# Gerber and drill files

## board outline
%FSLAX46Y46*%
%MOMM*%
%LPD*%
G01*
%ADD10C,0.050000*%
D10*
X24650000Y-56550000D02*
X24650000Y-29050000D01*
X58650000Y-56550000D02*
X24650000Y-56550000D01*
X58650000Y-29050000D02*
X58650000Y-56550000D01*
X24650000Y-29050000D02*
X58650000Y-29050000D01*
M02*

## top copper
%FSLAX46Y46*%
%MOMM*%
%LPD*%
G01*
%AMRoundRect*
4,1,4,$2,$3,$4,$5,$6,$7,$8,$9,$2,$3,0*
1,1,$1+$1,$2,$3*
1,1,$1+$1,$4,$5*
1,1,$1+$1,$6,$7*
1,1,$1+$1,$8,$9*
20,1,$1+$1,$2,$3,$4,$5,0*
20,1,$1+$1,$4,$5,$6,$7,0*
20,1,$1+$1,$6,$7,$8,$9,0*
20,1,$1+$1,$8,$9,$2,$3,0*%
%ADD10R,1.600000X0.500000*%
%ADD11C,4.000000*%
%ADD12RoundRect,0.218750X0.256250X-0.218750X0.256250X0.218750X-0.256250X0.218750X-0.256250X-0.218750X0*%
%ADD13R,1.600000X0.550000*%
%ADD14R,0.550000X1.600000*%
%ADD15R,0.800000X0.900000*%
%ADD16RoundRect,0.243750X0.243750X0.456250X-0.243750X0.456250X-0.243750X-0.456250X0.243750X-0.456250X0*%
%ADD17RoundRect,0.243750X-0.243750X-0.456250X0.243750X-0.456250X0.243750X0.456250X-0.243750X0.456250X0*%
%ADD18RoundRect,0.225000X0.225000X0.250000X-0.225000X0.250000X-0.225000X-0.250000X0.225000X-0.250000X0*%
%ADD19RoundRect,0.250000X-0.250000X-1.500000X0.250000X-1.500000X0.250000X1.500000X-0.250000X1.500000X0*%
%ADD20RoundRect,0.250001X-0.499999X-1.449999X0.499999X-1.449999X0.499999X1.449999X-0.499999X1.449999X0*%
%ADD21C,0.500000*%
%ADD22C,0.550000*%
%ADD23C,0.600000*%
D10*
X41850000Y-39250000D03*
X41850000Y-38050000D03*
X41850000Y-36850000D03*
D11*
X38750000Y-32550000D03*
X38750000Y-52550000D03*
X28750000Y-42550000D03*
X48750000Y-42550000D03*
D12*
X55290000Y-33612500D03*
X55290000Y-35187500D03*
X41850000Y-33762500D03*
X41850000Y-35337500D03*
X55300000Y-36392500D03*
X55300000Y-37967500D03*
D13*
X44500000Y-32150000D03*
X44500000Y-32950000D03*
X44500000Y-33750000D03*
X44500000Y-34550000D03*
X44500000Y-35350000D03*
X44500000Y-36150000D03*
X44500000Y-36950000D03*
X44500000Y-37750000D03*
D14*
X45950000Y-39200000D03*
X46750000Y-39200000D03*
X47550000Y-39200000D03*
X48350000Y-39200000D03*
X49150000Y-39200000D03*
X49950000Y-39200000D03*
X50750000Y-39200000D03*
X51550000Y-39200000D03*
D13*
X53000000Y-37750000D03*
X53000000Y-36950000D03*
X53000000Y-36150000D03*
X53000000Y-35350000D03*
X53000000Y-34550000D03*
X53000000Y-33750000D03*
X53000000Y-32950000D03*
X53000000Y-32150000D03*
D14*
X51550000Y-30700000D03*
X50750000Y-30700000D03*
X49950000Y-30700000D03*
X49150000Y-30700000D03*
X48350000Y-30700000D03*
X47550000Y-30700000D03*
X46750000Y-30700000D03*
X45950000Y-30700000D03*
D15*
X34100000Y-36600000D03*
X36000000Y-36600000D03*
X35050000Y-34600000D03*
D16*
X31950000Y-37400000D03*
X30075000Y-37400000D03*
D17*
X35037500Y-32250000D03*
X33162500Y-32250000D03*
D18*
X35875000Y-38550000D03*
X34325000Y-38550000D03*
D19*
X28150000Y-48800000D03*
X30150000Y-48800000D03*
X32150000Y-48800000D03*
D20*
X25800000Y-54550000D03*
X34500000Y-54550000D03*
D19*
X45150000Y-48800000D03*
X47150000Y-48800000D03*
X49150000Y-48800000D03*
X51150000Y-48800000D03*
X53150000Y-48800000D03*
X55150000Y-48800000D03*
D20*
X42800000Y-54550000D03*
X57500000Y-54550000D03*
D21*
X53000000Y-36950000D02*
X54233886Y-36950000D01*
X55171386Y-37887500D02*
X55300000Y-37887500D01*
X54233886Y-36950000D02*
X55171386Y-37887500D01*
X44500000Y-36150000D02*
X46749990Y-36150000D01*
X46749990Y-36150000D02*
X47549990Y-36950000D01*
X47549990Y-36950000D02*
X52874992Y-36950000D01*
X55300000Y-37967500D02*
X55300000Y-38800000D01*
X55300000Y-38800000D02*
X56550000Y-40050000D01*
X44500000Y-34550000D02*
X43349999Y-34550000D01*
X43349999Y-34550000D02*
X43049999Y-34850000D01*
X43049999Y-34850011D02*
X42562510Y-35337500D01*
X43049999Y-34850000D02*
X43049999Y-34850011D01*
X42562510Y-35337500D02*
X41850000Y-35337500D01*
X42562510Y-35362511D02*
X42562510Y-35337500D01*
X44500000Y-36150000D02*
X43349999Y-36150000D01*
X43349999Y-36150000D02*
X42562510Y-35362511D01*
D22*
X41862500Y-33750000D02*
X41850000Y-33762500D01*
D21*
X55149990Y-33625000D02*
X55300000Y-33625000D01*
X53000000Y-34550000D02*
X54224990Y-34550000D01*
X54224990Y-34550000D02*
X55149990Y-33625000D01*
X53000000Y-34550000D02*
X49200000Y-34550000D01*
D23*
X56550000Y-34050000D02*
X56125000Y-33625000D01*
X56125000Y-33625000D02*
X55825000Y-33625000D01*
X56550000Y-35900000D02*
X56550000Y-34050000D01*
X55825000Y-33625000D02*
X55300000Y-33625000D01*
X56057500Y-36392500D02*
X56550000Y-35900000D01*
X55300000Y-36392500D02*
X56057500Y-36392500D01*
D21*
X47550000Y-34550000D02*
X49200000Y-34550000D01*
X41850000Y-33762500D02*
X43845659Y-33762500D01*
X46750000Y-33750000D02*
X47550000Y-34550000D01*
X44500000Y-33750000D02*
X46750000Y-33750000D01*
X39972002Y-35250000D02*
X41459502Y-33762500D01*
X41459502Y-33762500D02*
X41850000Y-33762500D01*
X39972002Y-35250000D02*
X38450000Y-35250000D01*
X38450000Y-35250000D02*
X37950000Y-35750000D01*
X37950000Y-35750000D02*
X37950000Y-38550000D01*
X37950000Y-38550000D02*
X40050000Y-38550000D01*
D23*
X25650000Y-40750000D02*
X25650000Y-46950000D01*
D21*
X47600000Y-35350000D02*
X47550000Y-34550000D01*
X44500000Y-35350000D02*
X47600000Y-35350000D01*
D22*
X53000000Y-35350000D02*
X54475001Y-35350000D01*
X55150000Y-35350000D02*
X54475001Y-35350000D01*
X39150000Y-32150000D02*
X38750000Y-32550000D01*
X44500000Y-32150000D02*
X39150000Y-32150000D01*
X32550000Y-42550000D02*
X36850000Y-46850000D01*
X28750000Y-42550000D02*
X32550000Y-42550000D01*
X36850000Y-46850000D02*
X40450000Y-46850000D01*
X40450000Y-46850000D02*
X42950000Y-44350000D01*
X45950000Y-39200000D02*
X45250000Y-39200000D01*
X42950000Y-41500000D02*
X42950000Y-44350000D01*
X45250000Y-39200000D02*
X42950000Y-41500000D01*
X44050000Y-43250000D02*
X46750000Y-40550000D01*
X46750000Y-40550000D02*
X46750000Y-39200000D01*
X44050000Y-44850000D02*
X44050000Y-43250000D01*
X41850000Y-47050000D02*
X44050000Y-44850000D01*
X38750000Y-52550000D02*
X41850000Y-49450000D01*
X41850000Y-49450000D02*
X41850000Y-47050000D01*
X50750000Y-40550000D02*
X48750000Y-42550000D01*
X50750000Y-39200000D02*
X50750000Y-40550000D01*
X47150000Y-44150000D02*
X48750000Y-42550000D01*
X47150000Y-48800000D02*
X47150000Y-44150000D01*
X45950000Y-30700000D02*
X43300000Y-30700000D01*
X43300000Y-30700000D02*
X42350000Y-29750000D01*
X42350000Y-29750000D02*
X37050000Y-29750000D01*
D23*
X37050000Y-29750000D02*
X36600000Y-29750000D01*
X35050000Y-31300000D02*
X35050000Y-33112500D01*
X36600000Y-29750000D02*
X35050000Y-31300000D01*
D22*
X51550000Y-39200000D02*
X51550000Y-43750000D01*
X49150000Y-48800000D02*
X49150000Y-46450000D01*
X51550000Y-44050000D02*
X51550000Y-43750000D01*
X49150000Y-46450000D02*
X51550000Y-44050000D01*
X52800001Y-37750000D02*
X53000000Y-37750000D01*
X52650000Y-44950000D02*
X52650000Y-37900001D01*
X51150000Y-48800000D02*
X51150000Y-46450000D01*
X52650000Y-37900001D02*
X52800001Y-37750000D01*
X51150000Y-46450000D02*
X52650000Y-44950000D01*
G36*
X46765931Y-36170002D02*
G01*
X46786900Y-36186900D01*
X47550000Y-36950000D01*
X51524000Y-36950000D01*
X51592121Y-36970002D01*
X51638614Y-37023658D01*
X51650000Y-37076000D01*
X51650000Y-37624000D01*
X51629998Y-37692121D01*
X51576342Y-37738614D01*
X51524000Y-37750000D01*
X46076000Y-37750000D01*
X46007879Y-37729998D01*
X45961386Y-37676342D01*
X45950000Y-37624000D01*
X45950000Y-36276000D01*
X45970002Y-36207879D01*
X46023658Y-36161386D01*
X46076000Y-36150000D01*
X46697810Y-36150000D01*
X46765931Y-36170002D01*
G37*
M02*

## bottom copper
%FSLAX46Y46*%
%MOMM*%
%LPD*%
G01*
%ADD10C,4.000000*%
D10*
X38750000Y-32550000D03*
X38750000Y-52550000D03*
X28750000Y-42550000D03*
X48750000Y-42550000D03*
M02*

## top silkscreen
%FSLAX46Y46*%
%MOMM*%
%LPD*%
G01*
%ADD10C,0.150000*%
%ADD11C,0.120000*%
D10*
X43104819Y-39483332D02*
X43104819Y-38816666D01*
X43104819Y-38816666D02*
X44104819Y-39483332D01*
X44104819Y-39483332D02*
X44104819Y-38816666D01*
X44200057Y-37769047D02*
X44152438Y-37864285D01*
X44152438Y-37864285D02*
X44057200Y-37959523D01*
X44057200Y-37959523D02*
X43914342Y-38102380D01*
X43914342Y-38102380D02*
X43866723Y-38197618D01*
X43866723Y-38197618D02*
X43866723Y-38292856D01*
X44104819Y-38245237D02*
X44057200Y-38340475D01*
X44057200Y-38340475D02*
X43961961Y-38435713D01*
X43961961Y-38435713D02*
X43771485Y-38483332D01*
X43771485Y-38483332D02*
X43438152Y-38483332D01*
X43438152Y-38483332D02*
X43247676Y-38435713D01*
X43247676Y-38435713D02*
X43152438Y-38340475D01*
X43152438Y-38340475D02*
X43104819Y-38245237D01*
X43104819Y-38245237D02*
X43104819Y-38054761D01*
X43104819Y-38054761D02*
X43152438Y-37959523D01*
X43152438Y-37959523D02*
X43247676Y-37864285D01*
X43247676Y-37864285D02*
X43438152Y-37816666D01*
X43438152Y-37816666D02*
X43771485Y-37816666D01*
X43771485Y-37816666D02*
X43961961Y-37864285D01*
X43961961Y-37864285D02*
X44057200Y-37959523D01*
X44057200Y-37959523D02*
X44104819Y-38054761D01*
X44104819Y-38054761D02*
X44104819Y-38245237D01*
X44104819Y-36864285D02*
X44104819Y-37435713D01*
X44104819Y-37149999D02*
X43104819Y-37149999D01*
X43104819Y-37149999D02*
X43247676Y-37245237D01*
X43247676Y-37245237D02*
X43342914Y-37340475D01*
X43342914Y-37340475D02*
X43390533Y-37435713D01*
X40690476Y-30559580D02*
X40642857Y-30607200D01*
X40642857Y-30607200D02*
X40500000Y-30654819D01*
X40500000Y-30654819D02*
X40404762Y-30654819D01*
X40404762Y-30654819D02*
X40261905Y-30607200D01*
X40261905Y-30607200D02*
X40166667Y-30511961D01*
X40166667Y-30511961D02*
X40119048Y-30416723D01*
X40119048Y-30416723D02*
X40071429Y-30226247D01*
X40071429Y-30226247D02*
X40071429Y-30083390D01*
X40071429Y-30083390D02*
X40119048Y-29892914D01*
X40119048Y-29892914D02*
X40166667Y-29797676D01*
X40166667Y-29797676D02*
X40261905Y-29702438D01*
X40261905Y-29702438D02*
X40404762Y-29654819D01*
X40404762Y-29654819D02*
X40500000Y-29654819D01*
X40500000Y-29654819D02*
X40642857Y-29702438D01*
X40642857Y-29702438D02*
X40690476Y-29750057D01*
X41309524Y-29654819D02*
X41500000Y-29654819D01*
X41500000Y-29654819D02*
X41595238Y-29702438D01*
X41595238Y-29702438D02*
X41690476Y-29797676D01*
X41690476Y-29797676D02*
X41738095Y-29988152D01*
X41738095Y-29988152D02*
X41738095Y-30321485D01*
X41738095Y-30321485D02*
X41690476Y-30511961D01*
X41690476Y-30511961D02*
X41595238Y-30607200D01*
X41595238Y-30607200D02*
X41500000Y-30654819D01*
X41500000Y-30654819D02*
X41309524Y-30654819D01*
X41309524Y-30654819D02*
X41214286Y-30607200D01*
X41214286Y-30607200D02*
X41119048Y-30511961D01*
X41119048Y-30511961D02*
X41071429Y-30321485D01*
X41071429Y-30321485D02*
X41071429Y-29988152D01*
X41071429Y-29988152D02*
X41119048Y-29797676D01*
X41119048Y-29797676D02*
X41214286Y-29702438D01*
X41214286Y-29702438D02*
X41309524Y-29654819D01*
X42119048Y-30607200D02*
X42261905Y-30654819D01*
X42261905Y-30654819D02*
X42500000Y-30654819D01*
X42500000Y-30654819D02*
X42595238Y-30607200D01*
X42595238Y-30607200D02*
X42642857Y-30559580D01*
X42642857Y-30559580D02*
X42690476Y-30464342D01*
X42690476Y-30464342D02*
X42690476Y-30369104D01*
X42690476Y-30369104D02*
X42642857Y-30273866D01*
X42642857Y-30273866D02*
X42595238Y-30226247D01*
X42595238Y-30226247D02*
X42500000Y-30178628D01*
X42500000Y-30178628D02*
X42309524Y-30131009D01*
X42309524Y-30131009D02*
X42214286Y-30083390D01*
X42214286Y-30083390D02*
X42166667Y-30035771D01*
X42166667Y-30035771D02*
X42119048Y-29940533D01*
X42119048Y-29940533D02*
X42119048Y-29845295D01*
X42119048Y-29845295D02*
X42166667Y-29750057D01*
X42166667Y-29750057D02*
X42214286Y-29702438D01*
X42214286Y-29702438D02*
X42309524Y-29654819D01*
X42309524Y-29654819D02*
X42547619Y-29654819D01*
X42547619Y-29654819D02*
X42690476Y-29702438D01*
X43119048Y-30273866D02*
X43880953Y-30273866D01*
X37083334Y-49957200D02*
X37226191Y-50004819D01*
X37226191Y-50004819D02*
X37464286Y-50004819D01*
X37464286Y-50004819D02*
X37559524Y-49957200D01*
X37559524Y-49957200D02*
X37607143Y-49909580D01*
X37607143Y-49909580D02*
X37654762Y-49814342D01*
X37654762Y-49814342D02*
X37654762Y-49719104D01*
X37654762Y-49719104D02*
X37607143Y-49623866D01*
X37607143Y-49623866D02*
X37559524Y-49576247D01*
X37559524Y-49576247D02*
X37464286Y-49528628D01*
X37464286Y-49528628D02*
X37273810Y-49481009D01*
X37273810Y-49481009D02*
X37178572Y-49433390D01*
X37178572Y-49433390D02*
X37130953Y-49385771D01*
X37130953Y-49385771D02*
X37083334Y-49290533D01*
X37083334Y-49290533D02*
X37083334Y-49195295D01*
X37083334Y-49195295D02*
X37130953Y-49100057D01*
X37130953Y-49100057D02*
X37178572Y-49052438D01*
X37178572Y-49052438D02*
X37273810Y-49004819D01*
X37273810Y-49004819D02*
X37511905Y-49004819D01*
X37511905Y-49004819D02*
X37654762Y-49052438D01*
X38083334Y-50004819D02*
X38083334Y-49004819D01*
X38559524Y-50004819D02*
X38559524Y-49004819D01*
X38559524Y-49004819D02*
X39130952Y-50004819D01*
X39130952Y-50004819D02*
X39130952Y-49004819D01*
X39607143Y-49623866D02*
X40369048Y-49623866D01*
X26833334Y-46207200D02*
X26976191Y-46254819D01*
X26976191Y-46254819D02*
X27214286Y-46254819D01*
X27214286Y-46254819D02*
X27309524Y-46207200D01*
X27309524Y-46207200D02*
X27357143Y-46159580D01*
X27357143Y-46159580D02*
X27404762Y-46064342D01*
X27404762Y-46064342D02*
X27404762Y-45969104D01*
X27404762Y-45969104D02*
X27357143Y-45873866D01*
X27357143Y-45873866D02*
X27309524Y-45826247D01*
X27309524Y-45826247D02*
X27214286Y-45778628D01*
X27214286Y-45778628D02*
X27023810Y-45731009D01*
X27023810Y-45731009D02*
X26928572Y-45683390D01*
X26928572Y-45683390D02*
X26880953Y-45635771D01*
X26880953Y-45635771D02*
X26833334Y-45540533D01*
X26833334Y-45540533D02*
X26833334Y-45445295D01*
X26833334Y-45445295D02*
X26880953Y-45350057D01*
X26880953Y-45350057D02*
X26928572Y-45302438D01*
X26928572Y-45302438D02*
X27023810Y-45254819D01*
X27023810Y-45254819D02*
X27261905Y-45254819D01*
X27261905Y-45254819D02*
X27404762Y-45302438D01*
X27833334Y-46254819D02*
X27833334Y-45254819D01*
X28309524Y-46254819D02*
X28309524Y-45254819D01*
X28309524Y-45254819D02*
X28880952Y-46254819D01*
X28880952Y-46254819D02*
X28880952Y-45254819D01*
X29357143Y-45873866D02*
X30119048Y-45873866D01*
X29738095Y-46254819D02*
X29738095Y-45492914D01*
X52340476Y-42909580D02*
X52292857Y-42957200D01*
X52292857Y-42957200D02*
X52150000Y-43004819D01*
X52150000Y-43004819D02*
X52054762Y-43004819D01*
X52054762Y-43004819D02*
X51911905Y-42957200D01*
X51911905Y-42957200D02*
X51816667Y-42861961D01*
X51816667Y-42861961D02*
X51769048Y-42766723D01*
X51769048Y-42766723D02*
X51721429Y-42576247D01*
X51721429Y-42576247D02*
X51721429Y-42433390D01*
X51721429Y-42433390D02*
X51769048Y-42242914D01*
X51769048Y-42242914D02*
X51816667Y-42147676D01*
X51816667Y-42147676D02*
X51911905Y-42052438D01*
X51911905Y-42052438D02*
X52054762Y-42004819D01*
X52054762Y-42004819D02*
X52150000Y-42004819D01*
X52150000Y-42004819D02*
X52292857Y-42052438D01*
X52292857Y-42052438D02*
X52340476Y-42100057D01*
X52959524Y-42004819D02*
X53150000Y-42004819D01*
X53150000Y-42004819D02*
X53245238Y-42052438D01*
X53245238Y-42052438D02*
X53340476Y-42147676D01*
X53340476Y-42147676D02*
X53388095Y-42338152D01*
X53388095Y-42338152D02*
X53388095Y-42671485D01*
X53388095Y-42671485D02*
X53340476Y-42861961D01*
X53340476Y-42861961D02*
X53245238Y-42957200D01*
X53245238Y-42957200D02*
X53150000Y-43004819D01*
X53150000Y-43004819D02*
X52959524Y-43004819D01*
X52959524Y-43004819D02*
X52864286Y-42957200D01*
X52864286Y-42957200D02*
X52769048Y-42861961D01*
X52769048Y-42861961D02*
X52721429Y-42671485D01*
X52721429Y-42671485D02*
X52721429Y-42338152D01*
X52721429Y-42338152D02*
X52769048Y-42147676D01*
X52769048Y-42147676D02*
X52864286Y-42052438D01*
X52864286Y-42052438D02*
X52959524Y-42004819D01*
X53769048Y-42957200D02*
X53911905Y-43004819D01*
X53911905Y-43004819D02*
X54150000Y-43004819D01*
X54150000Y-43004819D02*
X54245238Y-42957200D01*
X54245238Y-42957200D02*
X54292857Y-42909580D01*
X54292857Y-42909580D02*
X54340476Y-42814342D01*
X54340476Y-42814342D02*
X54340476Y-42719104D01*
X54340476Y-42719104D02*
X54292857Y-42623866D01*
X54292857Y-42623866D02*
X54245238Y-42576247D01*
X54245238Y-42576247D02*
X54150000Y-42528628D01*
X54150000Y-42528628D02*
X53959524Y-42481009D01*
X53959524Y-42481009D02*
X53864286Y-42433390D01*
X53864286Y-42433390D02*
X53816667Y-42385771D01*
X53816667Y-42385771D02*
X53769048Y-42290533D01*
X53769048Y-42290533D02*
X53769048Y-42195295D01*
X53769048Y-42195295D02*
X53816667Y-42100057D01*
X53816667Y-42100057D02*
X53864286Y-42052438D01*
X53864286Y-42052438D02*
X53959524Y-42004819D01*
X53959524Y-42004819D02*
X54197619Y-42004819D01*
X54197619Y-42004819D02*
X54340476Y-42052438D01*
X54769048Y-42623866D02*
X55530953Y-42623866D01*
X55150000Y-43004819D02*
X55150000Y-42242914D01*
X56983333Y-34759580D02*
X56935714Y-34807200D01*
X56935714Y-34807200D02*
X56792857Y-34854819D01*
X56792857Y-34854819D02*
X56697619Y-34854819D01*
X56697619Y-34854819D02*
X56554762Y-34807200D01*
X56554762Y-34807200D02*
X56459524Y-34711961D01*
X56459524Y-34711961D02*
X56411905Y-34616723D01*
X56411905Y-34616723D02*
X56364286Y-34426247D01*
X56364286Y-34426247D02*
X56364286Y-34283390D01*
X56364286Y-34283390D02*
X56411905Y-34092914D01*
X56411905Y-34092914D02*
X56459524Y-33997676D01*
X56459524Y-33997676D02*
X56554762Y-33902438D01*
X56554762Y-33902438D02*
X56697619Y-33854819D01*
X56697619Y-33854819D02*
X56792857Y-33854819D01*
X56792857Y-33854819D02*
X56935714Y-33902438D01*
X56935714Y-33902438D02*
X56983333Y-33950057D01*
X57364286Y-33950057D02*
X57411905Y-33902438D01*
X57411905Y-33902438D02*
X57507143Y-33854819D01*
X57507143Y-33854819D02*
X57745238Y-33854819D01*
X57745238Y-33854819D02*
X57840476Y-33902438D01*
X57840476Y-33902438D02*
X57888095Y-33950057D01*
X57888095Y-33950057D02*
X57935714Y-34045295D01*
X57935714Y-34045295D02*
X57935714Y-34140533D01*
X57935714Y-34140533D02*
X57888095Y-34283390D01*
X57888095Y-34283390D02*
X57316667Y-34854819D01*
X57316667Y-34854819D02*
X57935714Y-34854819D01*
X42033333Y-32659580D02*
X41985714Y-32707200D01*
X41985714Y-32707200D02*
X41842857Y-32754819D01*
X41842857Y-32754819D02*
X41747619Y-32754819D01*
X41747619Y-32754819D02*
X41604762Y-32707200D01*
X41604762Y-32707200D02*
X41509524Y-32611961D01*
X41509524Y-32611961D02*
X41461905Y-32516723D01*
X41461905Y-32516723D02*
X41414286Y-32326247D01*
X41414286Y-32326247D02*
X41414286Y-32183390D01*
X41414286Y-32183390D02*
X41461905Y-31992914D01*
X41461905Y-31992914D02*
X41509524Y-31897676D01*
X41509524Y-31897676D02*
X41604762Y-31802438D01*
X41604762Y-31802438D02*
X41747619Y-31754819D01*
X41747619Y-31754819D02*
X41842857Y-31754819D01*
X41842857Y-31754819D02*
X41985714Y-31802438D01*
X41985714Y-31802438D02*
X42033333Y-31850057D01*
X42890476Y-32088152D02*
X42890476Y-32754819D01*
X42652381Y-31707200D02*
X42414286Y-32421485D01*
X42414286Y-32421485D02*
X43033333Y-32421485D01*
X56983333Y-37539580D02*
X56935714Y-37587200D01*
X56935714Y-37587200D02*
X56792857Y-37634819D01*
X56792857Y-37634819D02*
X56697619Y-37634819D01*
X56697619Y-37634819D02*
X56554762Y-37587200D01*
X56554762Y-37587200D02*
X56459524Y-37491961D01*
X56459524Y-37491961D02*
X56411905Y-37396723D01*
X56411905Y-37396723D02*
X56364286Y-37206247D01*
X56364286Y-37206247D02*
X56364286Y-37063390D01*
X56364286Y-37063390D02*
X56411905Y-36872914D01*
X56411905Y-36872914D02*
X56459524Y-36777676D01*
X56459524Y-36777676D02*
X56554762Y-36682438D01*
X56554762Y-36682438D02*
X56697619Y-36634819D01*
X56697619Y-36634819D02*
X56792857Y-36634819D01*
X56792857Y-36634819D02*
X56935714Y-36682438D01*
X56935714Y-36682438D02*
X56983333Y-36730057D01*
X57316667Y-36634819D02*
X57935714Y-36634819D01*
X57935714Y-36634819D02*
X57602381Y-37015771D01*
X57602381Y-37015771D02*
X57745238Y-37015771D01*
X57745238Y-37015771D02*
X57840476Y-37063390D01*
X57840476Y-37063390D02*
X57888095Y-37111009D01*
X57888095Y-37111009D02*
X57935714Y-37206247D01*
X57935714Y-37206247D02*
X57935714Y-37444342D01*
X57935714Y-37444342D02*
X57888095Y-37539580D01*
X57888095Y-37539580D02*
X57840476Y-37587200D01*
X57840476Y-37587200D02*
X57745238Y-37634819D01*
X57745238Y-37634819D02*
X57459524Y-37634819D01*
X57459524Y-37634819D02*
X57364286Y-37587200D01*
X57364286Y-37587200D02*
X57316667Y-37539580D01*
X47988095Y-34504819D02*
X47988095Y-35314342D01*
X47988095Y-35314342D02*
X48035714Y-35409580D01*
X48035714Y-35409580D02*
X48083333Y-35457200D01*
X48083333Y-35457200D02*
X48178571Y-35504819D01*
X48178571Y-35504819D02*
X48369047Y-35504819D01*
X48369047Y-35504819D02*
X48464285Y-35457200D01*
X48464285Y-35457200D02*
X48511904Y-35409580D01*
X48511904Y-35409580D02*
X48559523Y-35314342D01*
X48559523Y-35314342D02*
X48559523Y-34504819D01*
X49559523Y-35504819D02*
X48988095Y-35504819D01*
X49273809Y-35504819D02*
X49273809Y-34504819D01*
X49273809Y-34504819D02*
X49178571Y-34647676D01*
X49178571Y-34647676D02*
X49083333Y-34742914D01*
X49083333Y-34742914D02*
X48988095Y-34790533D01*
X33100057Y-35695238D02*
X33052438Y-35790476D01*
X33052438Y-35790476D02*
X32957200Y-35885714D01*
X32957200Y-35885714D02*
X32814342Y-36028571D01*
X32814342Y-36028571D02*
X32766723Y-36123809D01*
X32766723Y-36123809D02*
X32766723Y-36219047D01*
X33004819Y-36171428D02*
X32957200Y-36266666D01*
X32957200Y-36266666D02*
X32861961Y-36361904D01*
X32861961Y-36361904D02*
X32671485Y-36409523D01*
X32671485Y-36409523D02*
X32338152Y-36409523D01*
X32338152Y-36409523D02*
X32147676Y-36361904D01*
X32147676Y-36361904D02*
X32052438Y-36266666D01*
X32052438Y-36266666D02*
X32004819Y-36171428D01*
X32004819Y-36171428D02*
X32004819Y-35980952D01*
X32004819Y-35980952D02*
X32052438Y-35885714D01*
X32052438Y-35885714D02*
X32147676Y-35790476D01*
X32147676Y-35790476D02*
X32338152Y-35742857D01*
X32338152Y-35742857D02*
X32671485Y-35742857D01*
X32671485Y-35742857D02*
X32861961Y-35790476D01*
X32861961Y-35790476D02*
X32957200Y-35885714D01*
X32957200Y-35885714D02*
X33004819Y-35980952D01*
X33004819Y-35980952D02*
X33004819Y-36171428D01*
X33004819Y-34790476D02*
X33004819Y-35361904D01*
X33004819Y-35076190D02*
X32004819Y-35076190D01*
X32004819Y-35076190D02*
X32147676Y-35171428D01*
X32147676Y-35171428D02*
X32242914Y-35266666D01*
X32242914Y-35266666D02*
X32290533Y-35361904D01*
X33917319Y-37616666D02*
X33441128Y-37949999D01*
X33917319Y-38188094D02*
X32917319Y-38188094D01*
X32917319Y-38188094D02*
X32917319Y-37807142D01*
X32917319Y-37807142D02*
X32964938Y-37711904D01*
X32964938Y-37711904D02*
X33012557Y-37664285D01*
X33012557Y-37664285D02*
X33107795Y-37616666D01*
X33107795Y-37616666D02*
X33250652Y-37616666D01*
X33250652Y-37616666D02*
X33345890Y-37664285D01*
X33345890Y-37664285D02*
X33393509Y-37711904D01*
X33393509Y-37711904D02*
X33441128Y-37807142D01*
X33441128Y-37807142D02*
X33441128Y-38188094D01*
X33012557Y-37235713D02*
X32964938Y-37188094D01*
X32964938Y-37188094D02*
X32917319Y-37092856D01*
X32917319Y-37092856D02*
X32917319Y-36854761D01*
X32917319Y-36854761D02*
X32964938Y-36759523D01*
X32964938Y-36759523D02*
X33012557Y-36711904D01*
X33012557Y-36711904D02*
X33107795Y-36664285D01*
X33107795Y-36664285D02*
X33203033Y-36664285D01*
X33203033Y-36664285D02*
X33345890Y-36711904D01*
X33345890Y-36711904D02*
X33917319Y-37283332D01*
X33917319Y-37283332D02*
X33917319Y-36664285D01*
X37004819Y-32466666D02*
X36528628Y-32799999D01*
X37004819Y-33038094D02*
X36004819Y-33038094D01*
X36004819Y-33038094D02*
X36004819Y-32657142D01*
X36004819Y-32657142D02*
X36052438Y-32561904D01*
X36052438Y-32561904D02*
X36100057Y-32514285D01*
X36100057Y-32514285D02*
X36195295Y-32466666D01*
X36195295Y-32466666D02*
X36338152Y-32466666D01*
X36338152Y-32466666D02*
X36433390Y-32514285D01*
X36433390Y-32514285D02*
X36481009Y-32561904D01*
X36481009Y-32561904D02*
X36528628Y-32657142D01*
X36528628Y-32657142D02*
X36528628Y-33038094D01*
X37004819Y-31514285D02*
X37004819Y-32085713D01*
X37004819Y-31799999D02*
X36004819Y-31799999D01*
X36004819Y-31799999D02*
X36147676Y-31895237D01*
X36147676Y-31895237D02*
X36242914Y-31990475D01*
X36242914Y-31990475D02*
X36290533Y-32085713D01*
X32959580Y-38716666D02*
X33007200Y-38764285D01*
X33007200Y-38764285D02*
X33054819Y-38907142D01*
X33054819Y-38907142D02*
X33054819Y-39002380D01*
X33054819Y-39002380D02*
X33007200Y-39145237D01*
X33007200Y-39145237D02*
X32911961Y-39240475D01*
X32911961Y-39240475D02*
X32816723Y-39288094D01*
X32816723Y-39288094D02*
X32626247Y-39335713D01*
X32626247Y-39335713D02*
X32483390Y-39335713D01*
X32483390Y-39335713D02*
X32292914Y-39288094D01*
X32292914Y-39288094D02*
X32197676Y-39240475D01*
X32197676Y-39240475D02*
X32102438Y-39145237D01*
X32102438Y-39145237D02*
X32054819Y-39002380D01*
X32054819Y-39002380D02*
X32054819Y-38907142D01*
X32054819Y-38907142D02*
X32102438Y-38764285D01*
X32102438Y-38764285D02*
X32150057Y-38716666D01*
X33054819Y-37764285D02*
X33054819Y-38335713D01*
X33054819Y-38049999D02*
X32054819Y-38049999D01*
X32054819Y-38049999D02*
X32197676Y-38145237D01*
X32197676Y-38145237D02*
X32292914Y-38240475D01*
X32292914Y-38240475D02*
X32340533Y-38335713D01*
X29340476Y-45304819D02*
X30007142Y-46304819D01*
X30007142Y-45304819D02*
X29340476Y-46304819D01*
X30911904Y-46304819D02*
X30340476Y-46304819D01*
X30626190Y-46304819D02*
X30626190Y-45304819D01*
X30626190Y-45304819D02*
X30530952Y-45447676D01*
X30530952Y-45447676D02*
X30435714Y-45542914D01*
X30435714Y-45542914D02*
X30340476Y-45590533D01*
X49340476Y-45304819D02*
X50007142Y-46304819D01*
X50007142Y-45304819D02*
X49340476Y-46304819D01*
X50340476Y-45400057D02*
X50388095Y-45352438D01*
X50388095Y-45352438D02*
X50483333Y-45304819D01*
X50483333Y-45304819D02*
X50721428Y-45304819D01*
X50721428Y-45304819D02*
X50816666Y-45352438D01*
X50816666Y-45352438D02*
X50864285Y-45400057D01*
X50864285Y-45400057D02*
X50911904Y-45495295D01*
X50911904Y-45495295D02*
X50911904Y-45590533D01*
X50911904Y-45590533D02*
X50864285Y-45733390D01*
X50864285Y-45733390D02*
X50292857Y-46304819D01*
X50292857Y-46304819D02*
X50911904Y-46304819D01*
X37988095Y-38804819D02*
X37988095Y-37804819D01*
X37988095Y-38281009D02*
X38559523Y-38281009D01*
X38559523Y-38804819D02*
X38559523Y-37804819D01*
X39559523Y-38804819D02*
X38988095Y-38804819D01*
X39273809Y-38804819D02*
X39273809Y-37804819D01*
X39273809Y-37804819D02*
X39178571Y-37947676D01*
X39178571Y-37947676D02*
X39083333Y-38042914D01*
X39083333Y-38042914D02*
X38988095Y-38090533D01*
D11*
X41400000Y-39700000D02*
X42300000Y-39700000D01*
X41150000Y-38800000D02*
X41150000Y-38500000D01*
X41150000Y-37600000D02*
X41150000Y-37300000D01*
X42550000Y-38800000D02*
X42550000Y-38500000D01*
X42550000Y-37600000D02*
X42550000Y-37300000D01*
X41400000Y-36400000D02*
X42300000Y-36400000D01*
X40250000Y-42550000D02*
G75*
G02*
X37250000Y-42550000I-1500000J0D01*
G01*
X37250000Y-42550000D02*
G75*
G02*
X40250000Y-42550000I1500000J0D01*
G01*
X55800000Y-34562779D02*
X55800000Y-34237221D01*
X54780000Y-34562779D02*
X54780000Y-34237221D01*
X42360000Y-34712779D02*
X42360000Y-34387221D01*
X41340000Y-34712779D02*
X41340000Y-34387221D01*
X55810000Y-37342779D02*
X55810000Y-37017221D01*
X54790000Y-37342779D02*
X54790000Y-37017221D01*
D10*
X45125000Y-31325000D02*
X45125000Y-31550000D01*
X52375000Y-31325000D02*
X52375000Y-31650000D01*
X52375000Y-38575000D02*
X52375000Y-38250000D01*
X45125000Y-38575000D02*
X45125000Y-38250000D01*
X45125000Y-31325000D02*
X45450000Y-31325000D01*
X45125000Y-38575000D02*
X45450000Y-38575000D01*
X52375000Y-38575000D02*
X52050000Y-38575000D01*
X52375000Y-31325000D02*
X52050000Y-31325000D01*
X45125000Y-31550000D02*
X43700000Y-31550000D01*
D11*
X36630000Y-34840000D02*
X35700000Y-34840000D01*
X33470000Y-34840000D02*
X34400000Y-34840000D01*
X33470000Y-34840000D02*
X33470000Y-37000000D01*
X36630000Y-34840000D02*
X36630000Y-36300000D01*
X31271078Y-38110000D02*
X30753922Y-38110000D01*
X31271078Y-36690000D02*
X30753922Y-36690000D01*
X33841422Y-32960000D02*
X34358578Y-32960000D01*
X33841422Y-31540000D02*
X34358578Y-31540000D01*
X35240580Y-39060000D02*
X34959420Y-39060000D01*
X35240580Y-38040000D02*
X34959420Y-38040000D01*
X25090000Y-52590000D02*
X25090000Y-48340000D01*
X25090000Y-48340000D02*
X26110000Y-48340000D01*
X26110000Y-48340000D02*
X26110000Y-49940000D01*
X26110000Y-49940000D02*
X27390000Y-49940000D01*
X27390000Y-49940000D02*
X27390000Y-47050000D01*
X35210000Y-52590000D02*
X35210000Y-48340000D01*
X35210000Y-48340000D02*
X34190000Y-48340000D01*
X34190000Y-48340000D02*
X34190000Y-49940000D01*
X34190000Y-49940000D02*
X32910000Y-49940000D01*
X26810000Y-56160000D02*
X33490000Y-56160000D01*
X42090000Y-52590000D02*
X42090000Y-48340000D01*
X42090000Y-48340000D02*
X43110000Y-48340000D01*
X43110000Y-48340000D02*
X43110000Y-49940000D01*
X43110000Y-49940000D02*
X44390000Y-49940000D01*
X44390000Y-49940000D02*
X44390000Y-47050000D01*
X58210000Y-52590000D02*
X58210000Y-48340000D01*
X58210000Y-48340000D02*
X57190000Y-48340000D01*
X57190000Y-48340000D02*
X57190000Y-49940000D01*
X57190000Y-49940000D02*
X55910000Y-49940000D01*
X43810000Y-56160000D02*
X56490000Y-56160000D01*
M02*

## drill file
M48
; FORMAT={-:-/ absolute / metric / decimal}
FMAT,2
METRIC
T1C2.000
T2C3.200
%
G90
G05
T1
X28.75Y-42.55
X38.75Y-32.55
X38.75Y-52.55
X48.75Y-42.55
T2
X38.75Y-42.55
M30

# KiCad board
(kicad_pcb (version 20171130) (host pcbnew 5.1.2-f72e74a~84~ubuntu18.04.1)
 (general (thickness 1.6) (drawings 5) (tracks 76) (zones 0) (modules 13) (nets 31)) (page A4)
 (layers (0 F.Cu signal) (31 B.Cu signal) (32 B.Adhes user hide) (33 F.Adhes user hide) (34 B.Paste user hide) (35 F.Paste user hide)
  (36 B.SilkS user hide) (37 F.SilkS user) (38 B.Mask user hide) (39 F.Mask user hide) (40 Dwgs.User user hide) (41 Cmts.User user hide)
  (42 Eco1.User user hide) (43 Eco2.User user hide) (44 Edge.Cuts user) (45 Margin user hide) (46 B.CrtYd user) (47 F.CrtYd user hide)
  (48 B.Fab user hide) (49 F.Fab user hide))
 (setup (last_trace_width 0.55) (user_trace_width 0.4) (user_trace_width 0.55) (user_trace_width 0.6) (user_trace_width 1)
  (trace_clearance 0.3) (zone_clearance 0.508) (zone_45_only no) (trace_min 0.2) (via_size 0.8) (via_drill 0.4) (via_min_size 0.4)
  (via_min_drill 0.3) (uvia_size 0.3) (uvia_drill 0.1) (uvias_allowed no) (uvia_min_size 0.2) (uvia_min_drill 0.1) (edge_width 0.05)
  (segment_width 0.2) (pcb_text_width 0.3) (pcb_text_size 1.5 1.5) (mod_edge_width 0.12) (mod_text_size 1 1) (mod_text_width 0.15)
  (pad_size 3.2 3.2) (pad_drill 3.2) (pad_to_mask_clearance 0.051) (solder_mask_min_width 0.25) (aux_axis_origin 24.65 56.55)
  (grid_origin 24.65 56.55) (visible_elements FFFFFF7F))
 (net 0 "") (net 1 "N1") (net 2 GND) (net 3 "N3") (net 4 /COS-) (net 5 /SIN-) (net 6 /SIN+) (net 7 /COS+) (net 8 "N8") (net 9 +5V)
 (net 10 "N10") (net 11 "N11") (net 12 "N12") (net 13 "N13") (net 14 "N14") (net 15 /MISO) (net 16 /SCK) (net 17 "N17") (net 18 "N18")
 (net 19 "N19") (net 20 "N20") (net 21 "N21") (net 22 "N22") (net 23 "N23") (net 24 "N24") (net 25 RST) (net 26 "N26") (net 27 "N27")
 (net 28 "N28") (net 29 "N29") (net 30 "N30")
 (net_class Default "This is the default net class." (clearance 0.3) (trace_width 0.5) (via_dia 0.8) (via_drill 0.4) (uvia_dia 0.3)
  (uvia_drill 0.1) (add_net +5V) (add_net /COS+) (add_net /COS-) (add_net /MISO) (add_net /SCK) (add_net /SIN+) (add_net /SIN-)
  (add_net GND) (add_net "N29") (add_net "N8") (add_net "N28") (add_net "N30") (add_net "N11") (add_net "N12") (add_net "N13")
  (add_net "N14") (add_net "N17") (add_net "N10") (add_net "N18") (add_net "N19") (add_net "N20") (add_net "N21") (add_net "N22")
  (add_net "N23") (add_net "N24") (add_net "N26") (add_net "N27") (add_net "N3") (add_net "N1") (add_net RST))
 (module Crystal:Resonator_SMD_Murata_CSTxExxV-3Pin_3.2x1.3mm (layer F.Cu) (at 41.85 38.05 270)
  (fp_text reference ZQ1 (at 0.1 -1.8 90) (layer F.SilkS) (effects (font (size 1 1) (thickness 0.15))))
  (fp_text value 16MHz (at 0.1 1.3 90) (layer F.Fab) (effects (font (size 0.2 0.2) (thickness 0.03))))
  (fp_line (start 1.65 0.45) (end 1.65 -0.45) (layer F.SilkS) (width 0.12))
  (fp_line (start 0.75 0.7) (end 0.45 0.7) (layer F.SilkS) (width 0.12))
  (fp_line (start -0.45 0.7) (end -0.75 0.7) (layer F.SilkS) (width 0.12))
  (fp_line (start 0.75 -0.7) (end 0.45 -0.7) (layer F.SilkS) (width 0.12))
  (fp_line (start -0.45 -0.7) (end -0.75 -0.7) (layer F.SilkS) (width 0.12))
  (fp_line (start -1.65 0.45) (end -1.65 -0.45) (layer F.SilkS) (width 0.12))
  (pad 3 smd rect (at 1.2 0 270) (size 0.5 1.6) (layers F.Cu F.Paste F.Mask) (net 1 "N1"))
  (pad 2 smd rect (at 0 0 270) (size 0.5 1.6) (layers F.Cu F.Paste F.Mask) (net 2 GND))
  (pad 1 smd rect (at -1.2 0 270) (size 0.5 1.6) (layers F.Cu F.Paste F.Mask) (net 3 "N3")))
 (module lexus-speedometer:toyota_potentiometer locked (layer F.Cu) (at 38.75 42.55)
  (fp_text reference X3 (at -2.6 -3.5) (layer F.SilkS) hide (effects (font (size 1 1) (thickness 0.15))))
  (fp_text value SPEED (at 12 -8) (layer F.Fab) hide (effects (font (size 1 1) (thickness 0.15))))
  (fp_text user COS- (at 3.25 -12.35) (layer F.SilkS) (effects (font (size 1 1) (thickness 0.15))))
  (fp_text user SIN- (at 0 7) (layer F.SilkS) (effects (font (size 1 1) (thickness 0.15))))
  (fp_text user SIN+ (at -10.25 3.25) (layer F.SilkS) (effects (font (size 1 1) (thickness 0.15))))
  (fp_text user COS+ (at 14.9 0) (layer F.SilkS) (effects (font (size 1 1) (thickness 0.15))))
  (fp_circle (center 0 0) (end 1.5 0) (layer F.SilkS) (width 0.12))
  (pad 4 thru_hole circle (at 0 -10) (size 4 4) (drill 2) (layers F.Cu F.Mask) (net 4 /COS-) (clearance 0.6))
  (pad 2 thru_hole circle (at 0 10) (size 4 4) (drill 2) (layers F.Cu F.Mask) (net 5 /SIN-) (clearance 0.6))
  (pad 1 thru_hole circle (at -10 0) (size 4 4) (drill 2) (layers F.Cu F.Mask) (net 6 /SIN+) (clearance 0.6))
  (pad 3 thru_hole circle (at 10 0) (size 4 4) (drill 2) (layers F.Cu F.Mask) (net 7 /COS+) (clearance 0.6)))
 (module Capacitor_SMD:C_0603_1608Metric (layer F.Cu) (at 55.29 34.4 90)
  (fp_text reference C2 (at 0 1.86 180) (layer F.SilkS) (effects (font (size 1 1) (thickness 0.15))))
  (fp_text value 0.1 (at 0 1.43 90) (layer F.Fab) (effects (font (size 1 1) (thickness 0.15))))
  (fp_line (start -0.162779 0.51) (end 0.162779 0.51) (layer F.SilkS) (width 0.12))
  (fp_line (start -0.162779 -0.51) (end 0.162779 -0.51) (layer F.SilkS) (width 0.12))
  (pad 2 smd roundrect (at 0.7875 0 90) (size 0.875 0.95) (layers F.Cu F.Paste F.Mask) (roundrect_rratio 0.25) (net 2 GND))
  (pad 1 smd roundrect (at -0.7875 0 90) (size 0.875 0.95) (layers F.Cu F.Paste F.Mask) (roundrect_rratio 0.25) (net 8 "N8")))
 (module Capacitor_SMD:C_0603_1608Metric (layer F.Cu) (at 41.85 34.55 90)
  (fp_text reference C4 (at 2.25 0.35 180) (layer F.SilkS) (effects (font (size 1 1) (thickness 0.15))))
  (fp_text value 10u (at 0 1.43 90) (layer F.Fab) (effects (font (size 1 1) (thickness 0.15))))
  (fp_line (start -0.162779 0.51) (end 0.162779 0.51) (layer F.SilkS) (width 0.12))
  (fp_line (start -0.162779 -0.51) (end 0.162779 -0.51) (layer F.SilkS) (width 0.12))
  (pad 2 smd roundrect (at 0.7875 0 90) (size 0.875 0.95) (layers F.Cu F.Paste F.Mask) (roundrect_rratio 0.25) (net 2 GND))
  (pad 1 smd roundrect (at -0.7875 0 90) (size 0.875 0.95) (layers F.Cu F.Paste F.Mask) (roundrect_rratio 0.25) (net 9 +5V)))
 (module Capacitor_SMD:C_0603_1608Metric (layer F.Cu) (at 55.3 37.18 90)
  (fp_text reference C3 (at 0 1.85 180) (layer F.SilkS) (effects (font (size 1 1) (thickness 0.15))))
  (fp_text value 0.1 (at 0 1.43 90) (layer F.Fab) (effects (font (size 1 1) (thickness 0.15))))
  (fp_line (start -0.162779 0.51) (end 0.162779 0.51) (layer F.SilkS) (width 0.12))
  (fp_line (start -0.162779 -0.51) (end 0.162779 -0.51) (layer F.SilkS) (width 0.12))
  (pad 2 smd roundrect (at 0.7875 0 90) (size 0.875 0.95) (layers F.Cu F.Paste F.Mask) (roundrect_rratio 0.25) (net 2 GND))
  (pad 1 smd roundrect (at -0.7875 0 90) (size 0.875 0.95) (layers F.Cu F.Paste F.Mask) (roundrect_rratio 0.25) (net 9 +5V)))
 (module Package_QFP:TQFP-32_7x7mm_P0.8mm (layer F.Cu) (at 48.75 34.95)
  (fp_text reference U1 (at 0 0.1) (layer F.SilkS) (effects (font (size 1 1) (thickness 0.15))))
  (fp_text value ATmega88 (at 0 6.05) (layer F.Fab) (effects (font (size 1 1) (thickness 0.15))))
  (fp_line (start -3.625 -3.625) (end -3.625 -3.4) (layer F.SilkS) (width 0.15))
  (fp_line (start 3.625 -3.625) (end 3.625 -3.3) (layer F.SilkS) (width 0.15))
  (fp_line (start 3.625 3.625) (end 3.625 3.3) (layer F.SilkS) (width 0.15))
  (fp_line (start -3.625 3.625) (end -3.625 3.3) (layer F.SilkS) (width 0.15))
  (fp_line (start -3.625 -3.625) (end -3.3 -3.625) (layer F.SilkS) (width 0.15))
  (fp_line (start -3.625 3.625) (end -3.3 3.625) (layer F.SilkS) (width 0.15))
  (fp_line (start 3.625 3.625) (end 3.3 3.625) (layer F.SilkS) (width 0.15))
  (fp_line (start 3.625 -3.625) (end 3.3 -3.625) (layer F.SilkS) (width 0.15))
  (fp_line (start -3.625 -3.4) (end -5.05 -3.4) (layer F.SilkS) (width 0.15))
  (pad 1 smd rect (at -4.25 -2.8) (size 1.6 0.55) (layers F.Cu F.Paste F.Mask) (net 4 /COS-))
  (pad 2 smd rect (at -4.25 -2) (size 1.6 0.55) (layers F.Cu F.Paste F.Mask) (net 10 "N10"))
  (pad 3 smd rect (at -4.25 -1.2) (size 1.6 0.55) (layers F.Cu F.Paste F.Mask) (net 2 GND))
  (pad 4 smd rect (at -4.25 -0.4) (size 1.6 0.55) (layers F.Cu F.Paste F.Mask) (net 9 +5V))
  (pad 5 smd rect (at -4.25 0.4) (size 1.6 0.55) (layers F.Cu F.Paste F.Mask) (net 2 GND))
  (pad 6 smd rect (at -4.25 1.2) (size 1.6 0.55) (layers F.Cu F.Paste F.Mask) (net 9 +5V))
  (pad 7 smd rect (at -4.25 2) (size 1.6 0.55) (layers F.Cu F.Paste F.Mask) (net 3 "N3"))
  (pad 8 smd rect (at -4.25 2.8) (size 1.6 0.55) (layers F.Cu F.Paste F.Mask) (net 1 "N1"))
  (pad 9 smd rect (at -2.8 4.25 90) (size 1.6 0.55) (layers F.Cu F.Paste F.Mask) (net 6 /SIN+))
  (pad 10 smd rect (at -2 4.25 90) (size 1.6 0.55) (layers F.Cu F.Paste F.Mask) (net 5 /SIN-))
  (pad 11 smd rect (at -1.2 4.25 90) (size 1.6 0.55) (layers F.Cu F.Paste F.Mask) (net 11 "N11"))
  (pad 12 smd rect (at -0.4 4.25 90) (size 1.6 0.55) (layers F.Cu F.Paste F.Mask) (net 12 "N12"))
  (pad 13 smd rect (at 0.4 4.25 90) (size 1.6 0.55) (layers F.Cu F.Paste F.Mask) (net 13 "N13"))
  (pad 14 smd rect (at 1.2 4.25 90) (size 1.6 0.55) (layers F.Cu F.Paste F.Mask) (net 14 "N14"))
  (pad 15 smd rect (at 2 4.25 90) (size 1.6 0.55) (layers F.Cu F.Paste F.Mask) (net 7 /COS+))
  (pad 16 smd rect (at 2.8 4.25 90) (size 1.6 0.55) (layers F.Cu F.Paste F.Mask) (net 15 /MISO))
  (pad 17 smd rect (at 4.25 2.8) (size 1.6 0.55) (layers F.Cu F.Paste F.Mask) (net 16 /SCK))
  (pad 18 smd rect (at 4.25 2) (size 1.6 0.55) (layers F.Cu F.Paste F.Mask) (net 9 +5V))
  (pad 19 smd rect (at 4.25 1.2) (size 1.6 0.55) (layers F.Cu F.Paste F.Mask) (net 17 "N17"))
  (pad 20 smd rect (at 4.25 0.4) (size 1.6 0.55) (layers F.Cu F.Paste F.Mask) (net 8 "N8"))
  (pad 21 smd rect (at 4.25 -0.4) (size 1.6 0.55) (layers F.Cu F.Paste F.Mask) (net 2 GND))
  (pad 22 smd rect (at 4.25 -1.2) (size 1.6 0.55) (layers F.Cu F.Paste F.Mask) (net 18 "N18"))
  (pad 23 smd rect (at 4.25 -2) (size 1.6 0.55) (layers F.Cu F.Paste F.Mask) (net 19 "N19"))
  (pad 24 smd rect (at 4.25 -2.8) (size 1.6 0.55) (layers F.Cu F.Paste F.Mask) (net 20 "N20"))
  (pad 25 smd rect (at 2.8 -4.25 90) (size 1.6 0.55) (layers F.Cu F.Paste F.Mask) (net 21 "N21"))
  (pad 26 smd rect (at 2 -4.25 90) (size 1.6 0.55) (layers F.Cu F.Paste F.Mask) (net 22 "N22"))
  (pad 27 smd rect (at 1.2 -4.25 90) (size 1.6 0.55) (layers F.Cu F.Paste F.Mask) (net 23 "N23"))
  (pad 28 smd rect (at 0.4 -4.25 90) (size 1.6 0.55) (layers F.Cu F.Paste F.Mask) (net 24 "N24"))
  (pad 29 smd rect (at -0.4 -4.25 90) (size 1.6 0.55) (layers F.Cu F.Paste F.Mask) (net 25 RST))
  (pad 30 smd rect (at -1.2 -4.25 90) (size 1.6 0.55) (layers F.Cu F.Paste F.Mask) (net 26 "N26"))
  (pad 31 smd rect (at -2 -4.25 90) (size 1.6 0.55) (layers F.Cu F.Paste F.Mask) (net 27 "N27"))
  (pad 32 smd rect (at -2.8 -4.25 90) (size 1.6 0.55) (layers F.Cu F.Paste F.Mask) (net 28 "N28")))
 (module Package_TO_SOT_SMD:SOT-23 (layer F.Cu) (at 35.05 35.6 90)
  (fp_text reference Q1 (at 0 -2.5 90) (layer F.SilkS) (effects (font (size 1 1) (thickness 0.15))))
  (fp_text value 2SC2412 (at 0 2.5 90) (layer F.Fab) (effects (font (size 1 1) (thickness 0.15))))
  (fp_line (start 0.76 1.58) (end 0.76 0.65) (layer F.SilkS) (width 0.12))
  (fp_line (start 0.76 -1.58) (end 0.76 -0.65) (layer F.SilkS) (width 0.12))
  (fp_line (start 0.76 -1.58) (end -1.4 -1.58) (layer F.SilkS) (width 0.12))
  (fp_line (start 0.76 1.58) (end -0.7 1.58) (layer F.SilkS) (width 0.12))
  (pad 1 smd rect (at -1 -0.95 90) (size 0.9 0.8) (layers F.Cu F.Paste F.Mask) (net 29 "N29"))
  (pad 2 smd rect (at -1 0.95 90) (size 0.9 0.8) (layers F.Cu F.Paste F.Mask) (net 2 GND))
  (pad 3 smd rect (at 1 0 90) (size 0.9 0.8) (layers F.Cu F.Paste F.Mask) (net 28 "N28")))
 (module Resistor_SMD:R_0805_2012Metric (layer F.Cu) (at 31.0125 37.4 180)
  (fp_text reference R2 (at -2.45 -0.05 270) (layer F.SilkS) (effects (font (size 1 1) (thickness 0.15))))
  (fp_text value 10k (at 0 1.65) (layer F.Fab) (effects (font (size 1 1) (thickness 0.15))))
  (fp_line (start -0.258578 -0.71) (end 0.258578 -0.71) (layer F.SilkS) (width 0.12))
  (fp_line (start -0.258578 0.71) (end 0.258578 0.71) (layer F.SilkS) (width 0.12))
  (pad 1 smd roundrect (at -0.9375 0 180) (size 0.975 1.4) (layers F.Cu F.Paste F.Mask) (roundrect_rratio 0.25) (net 29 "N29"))
  (pad 2 smd roundrect (at 0.9375 0 180) (size 0.975 1.4) (layers F.Cu F.Paste F.Mask) (roundrect_rratio 0.25) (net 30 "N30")))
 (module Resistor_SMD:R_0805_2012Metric (layer F.Cu) (at 34.1 32.25)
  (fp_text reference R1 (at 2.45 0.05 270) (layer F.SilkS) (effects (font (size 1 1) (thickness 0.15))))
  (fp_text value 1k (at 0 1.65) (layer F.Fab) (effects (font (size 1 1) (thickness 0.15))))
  (fp_line (start -0.258578 0.71) (end 0.258578 0.71) (layer F.SilkS) (width 0.12))
  (fp_line (start -0.258578 -0.71) (end 0.258578 -0.71) (layer F.SilkS) (width 0.12))
  (pad 2 smd roundrect (at 0.9375 0) (size 0.975 1.4) (layers F.Cu F.Paste F.Mask) (roundrect_rratio 0.25) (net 28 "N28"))
  (pad 1 smd roundrect (at -0.9375 0) (size 0.975 1.4) (layers F.Cu F.Paste F.Mask) (roundrect_rratio 0.25) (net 9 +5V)))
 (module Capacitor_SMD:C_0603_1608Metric (layer F.Cu) (at 35.1 38.55 180)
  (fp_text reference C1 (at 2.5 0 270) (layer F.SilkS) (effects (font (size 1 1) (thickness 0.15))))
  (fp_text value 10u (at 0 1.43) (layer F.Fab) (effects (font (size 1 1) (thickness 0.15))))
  (fp_line (start -0.14058 -0.51) (end 0.14058 -0.51) (layer F.SilkS) (width 0.12))
  (fp_line (start -0.14058 0.51) (end 0.14058 0.51) (layer F.SilkS) (width 0.12))
  (pad 1 smd roundrect (at -0.775 0 180) (size 0.9 0.95) (layers F.Cu F.Paste F.Mask) (roundrect_rratio 0.25) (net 2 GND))
  (pad 2 smd roundrect (at 0.775 0 180) (size 0.9 0.95) (layers F.Cu F.Paste F.Mask) (roundrect_rratio 0.25) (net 29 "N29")))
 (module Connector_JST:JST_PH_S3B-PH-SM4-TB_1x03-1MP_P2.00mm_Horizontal (layer F.Cu) (at 30.15 51.65)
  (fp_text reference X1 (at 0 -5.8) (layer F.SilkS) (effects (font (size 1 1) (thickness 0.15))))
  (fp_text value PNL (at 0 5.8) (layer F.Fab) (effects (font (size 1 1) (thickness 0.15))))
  (fp_line (start -5.06 0.94) (end -5.06 -3.31) (layer F.SilkS) (width 0.12))
  (fp_line (start -5.06 -3.31) (end -4.04 -3.31) (layer F.SilkS) (width 0.12))
  (fp_line (start -4.04 -3.31) (end -4.04 -1.71) (layer F.SilkS) (width 0.12))
  (fp_line (start -4.04 -1.71) (end -2.76 -1.71) (layer F.SilkS) (width 0.12))
  (fp_line (start -2.76 -1.71) (end -2.76 -4.6) (layer F.SilkS) (width 0.12))
  (fp_line (start 5.06 0.94) (end 5.06 -3.31) (layer F.SilkS) (width 0.12))
  (fp_line (start 5.06 -3.31) (end 4.04 -3.31) (layer F.SilkS) (width 0.12))
  (fp_line (start 4.04 -3.31) (end 4.04 -1.71) (layer F.SilkS) (width 0.12))
  (fp_line (start 4.04 -1.71) (end 2.76 -1.71) (layer F.SilkS) (width 0.12))
  (fp_line (start -3.34 4.51) (end 3.34 4.51) (layer F.SilkS) (width 0.12))
  (pad 1 smd roundrect (at -2 -2.85) (size 1 3.5) (layers F.Cu F.Paste F.Mask) (roundrect_rratio 0.25) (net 2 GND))
  (pad 2 smd roundrect (at 0 -2.85) (size 1 3.5) (layers F.Cu F.Paste F.Mask) (roundrect_rratio 0.25) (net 30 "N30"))
  (pad 3 smd roundrect (at 2 -2.85) (size 1 3.5) (layers F.Cu F.Paste F.Mask) (roundrect_rratio 0.25) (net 9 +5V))
  (pad MP smd roundrect (at -4.35 2.9) (size 1.5 3.4) (layers F.Cu F.Paste F.Mask) (roundrect_rratio 0.166667))
  (pad MP smd roundrect (at 4.35 2.9) (size 1.5 3.4) (layers F.Cu F.Paste F.Mask) (roundrect_rratio 0.166667)))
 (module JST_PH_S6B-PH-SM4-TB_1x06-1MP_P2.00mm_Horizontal (layer F.Cu) (at 50.15 51.65)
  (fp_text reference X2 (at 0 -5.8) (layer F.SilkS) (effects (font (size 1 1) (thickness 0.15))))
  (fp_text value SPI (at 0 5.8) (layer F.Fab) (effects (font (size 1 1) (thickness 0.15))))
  (fp_line (start -8.06 0.94) (end -8.06 -3.31) (layer F.SilkS) (width 0.12))
  (fp_line (start -8.06 -3.31) (end -7.04 -3.31) (layer F.SilkS) (width 0.12))
  (fp_line (start -7.04 -3.31) (end -7.04 -1.71) (layer F.SilkS) (width 0.12))
  (fp_line (start -7.04 -1.71) (end -5.76 -1.71) (layer F.SilkS) (width 0.12))
  (fp_line (start -5.76 -1.71) (end -5.76 -4.6) (layer F.SilkS) (width 0.12))
  (fp_line (start 8.06 0.94) (end 8.06 -3.31) (layer F.SilkS) (width 0.12))
  (fp_line (start 8.06 -3.31) (end 7.04 -3.31) (layer F.SilkS) (width 0.12))
  (fp_line (start 7.04 -3.31) (end 7.04 -1.71) (layer F.SilkS) (width 0.12))
  (fp_line (start 7.04 -1.71) (end 5.76 -1.71) (layer F.SilkS) (width 0.12))
  (fp_line (start -6.34 4.51) (end 6.34 4.51) (layer F.SilkS) (width 0.12))
  (pad 1 smd roundrect (at -5 -2.85) (size 1 3.5) (layers F.Cu F.Paste F.Mask) (roundrect_rratio 0.25) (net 2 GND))
  (pad 2 smd roundrect (at -3 -2.85) (size 1 3.5) (layers F.Cu F.Paste F.Mask) (roundrect_rratio 0.25) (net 7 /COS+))
  (pad 3 smd roundrect (at -1 -2.85) (size 1 3.5) (layers F.Cu F.Paste F.Mask) (roundrect_rratio 0.25) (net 15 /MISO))
  (pad 4 smd roundrect (at 1 -2.85) (size 1 3.5) (layers F.Cu F.Paste F.Mask) (roundrect_rratio 0.25) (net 16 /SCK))
  (pad 5 smd roundrect (at 3 -2.85) (size 1 3.5) (layers F.Cu F.Paste F.Mask) (roundrect_rratio 0.25) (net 25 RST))
  (pad 6 smd roundrect (at 5 -2.85) (size 1 3.5) (layers F.Cu F.Paste F.Mask) (roundrect_rratio 0.25) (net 9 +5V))
  (pad MP smd roundrect (at -7.35 2.9) (size 1.5 3.4) (layers F.Cu F.Paste F.Mask) (roundrect_rratio 0.166667))
  (pad MP smd roundrect (at 7.35 2.9) (size 1.5 3.4) (layers F.Cu F.Paste F.Mask) (roundrect_rratio 0.166667)))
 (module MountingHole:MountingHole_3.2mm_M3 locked (layer F.Cu) (at 38.75 42.55) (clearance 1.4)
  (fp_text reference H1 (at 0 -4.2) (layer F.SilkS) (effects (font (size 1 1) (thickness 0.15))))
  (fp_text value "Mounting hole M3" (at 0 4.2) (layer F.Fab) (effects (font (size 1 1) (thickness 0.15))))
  (pad 1 np_thru_hole circle (at 0 0) (size 3.2 3.2) (drill 3.2) (layers *.Cu *.Mask)))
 (gr_line (start 24.65 56.55) (end 24.65 29.05) (layer Edge.Cuts) (width 0.05))
 (gr_line (start 58.65 56.55) (end 24.65 56.55) (layer Edge.Cuts) (width 0.05))
 (gr_line (start 58.65 29.05) (end 58.65 56.55) (layer Edge.Cuts) (width 0.05))
 (gr_line (start 24.65 29.05) (end 58.65 29.05) (layer Edge.Cuts) (width 0.05))
 (segment (start 53 36.95) (end 54.233886 36.95) (width 0.5) (layer F.Cu) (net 9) (status 10))
 (segment (start 55.171386 37.8875) (end 55.3 37.8875) (width 0.5) (layer F.Cu) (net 9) (status 30))
 (segment (start 54.233886 36.95) (end 55.171386 37.8875) (width 0.5) (layer F.Cu) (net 9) (status 20))
 (segment (start 44.5 36.15) (end 46.74999 36.15) (width 0.5) (layer F.Cu) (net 9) (status 10))
 (segment (start 46.74999 36.15) (end 47.54999 36.95) (width 0.5) (layer F.Cu) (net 9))
 (segment (start 47.54999 36.95) (end 52.874992 36.95) (width 0.5) (layer F.Cu) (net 9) (status 20))
 (segment (start 55.3 37.9675) (end 55.3 38.8) (width 0.5) (layer F.Cu) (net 9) (status 10))
 (segment (start 55.3 38.8) (end 56.55 40.05) (width 0.5) (layer F.Cu) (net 9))
 (segment (start 44.5 34.55) (end 43.349999 34.55) (width 0.5) (layer F.Cu) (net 9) (status 10))
 (segment (start 43.349999 34.55) (end 43.049999 34.85) (width 0.5) (layer F.Cu) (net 9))
 (segment (start 43.049999 34.850011) (end 42.56251 35.3375) (width 0.5) (layer F.Cu) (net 9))
 (segment (start 43.049999 34.85) (end 43.049999 34.850011) (width 0.5) (layer F.Cu) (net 9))
 (segment (start 42.56251 35.3375) (end 41.85 35.3375) (width 0.5) (layer F.Cu) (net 9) (status 20))
 (segment (start 42.56251 35.362511) (end 42.56251 35.3375) (width 0.5) (layer F.Cu) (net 9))
 (segment (start 44.5 36.15) (end 43.349999 36.15) (width 0.5) (layer F.Cu) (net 9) (status 10))
 (segment (start 43.349999 36.15) (end 42.56251 35.362511) (width 0.5) (layer F.Cu) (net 9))
 (segment (start 41.8625 33.75) (end 41.85 33.7625) (width 0.55) (layer F.Cu) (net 2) (status 30))
 (segment (start 55.14999 33.625) (end 55.3 33.625) (width 0.5) (layer F.Cu) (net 2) (status 30))
 (segment (start 53 34.55) (end 54.22499 34.55) (width 0.5) (layer F.Cu) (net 2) (status 10))
 (segment (start 54.22499 34.55) (end 55.14999 33.625) (width 0.5) (layer F.Cu) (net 2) (status 20))
 (segment (start 53 34.55) (end 49.2 34.55) (width 0.5) (layer F.Cu) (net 2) (status 10))
 (segment (start 56.55 34.05) (end 56.125 33.625) (width 0.6) (layer F.Cu) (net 2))
 (segment (start 56.125 33.625) (end 55.825 33.625) (width 0.6) (layer F.Cu) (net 2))
 (segment (start 56.55 35.9) (end 56.55 34.05) (width 0.6) (layer F.Cu) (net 2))
 (segment (start 55.825 33.625) (end 55.3 33.625) (width 0.6) (layer F.Cu) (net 2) (status 20))
 (segment (start 56.0575 36.3925) (end 56.55 35.9) (width 0.6) (layer F.Cu) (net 2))
 (segment (start 55.3 36.3925) (end 56.0575 36.3925) (width 0.6) (layer F.Cu) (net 2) (status 10))
 (segment (start 47.55 34.55) (end 49.2 34.55) (width 0.5) (layer F.Cu) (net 2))
 (segment (start 41.85 33.7625) (end 43.845659 33.7625) (width 0.5) (layer F.Cu) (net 2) (status 30))
 (segment (start 46.75 33.75) (end 47.55 34.55) (width 0.5) (layer F.Cu) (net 2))
 (segment (start 44.5 33.75) (end 46.75 33.75) (width 0.5) (layer F.Cu) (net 2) (status 10))
 (segment (start 39.972002 35.25) (end 41.459502 33.7625) (width 0.5) (layer F.Cu) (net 2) (status 20))
 (segment (start 41.459502 33.7625) (end 41.85 33.7625) (width 0.5) (layer F.Cu) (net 2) (status 30))
 (segment (start 39.972002 35.25) (end 38.45 35.25) (width 0.5) (layer F.Cu) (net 2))
 (segment (start 38.45 35.25) (end 37.95 35.75) (width 0.5) (layer F.Cu) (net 2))
 (segment (start 37.95 35.75) (end 37.95 38.55) (width 0.5) (layer F.Cu) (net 2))
 (segment (start 37.95 38.55) (end 40.05 38.55) (width 0.5) (layer F.Cu) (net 2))
 (segment (start 25.65 40.75) (end 25.65 46.95) (width 0.6) (layer F.Cu) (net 2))
 (segment (start 47.6 35.35) (end 47.55 34.55) (width 0.5) (layer F.Cu) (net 2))
 (segment (start 44.5 35.35) (end 47.6 35.35) (width 0.5) (layer F.Cu) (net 2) (status 10))
 (segment (start 53 35.35) (end 54.475001 35.35) (width 0.55) (layer F.Cu) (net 8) (status 10))
 (segment (start 55.15 35.35) (end 54.475001 35.35) (width 0.55) (layer F.Cu) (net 8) (status 10))
 (segment (start 39.15 32.15) (end 38.75 32.55) (width 0.55) (layer F.Cu) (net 4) (status 30))
 (segment (start 44.5 32.15) (end 39.15 32.15) (width 0.55) (layer F.Cu) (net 4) (status 30))
 (segment (start 32.55 42.55) (end 36.85 46.85) (width 0.55) (layer F.Cu) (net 6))
 (segment (start 28.75 42.55) (end 32.55 42.55) (width 0.55) (layer F.Cu) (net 6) (status 10))
 (segment (start 36.85 46.85) (end 40.45 46.85) (width 0.55) (layer F.Cu) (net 6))
 (segment (start 40.45 46.85) (end 42.95 44.35) (width 0.55) (layer F.Cu) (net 6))
 (segment (start 45.95 39.2) (end 45.25 39.2) (width 0.55) (layer F.Cu) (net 6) (status 10))
 (segment (start 42.95 41.5) (end 42.95 44.35) (width 0.55) (layer F.Cu) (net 6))
 (segment (start 45.25 39.2) (end 42.95 41.5) (width 0.55) (layer F.Cu) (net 6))
 (segment (start 44.05 43.25) (end 46.75 40.55) (width 0.55) (layer F.Cu) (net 5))
 (segment (start 46.75 40.55) (end 46.75 39.2) (width 0.55) (layer F.Cu) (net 5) (status 20))
 (segment (start 44.05 44.85) (end 44.05 43.25) (width 0.55) (layer F.Cu) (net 5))
 (segment (start 41.85 47.05) (end 44.05 44.85) (width 0.55) (layer F.Cu) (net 5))
 (segment (start 38.75 52.55) (end 41.85 49.45) (width 0.55) (layer F.Cu) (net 5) (status 10))
 (segment (start 41.85 49.45) (end 41.85 47.05) (width 0.55) (layer F.Cu) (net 5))
 (segment (start 50.75 40.55) (end 48.75 42.55) (width 0.55) (layer F.Cu) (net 7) (status 20))
 (segment (start 50.75 39.2) (end 50.75 40.55) (width 0.55) (layer F.Cu) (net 7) (status 10))
 (segment (start 47.15 44.15) (end 48.75 42.55) (width 0.55) (layer F.Cu) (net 7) (status 20))
 (segment (start 47.15 48.8) (end 47.15 44.15) (width 0.55) (layer F.Cu) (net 7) (status 10))
 (segment (start 45.95 30.7) (end 43.3 30.7) (width 0.55) (layer F.Cu) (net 28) (status 10))
 (segment (start 43.3 30.7) (end 42.35 29.75) (width 0.55) (layer F.Cu) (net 28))
 (segment (start 42.35 29.75) (end 37.05 29.75) (width 0.55) (layer F.Cu) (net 28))
 (segment (start 37.05 29.75) (end 36.6 29.75) (width 0.6) (layer F.Cu) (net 28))
 (segment (start 35.05 31.3) (end 35.05 33.1125) (width 0.6) (layer F.Cu) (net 28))
 (segment (start 36.6 29.75) (end 35.05 31.3) (width 0.6) (layer F.Cu) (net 28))
 (segment (start 51.55 39.2) (end 51.55 43.75) (width 0.55) (layer F.Cu) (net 15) (status 10))
 (segment (start 49.15 48.8) (end 49.15 46.45) (width 0.55) (layer F.Cu) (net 15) (status 10))
 (segment (start 51.55 44.05) (end 51.55 43.75) (width 0.55) (layer F.Cu) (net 15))
 (segment (start 49.15 46.45) (end 51.55 44.05) (width 0.55) (layer F.Cu) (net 15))
 (segment (start 52.800001 37.75) (end 53 37.75) (width 0.55) (layer F.Cu) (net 16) (status 30))
 (segment (start 52.65 44.95) (end 52.65 37.900001) (width 0.55) (layer F.Cu) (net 16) (status 20))
 (segment (start 51.15 48.8) (end 51.15 46.45) (width 0.55) (layer F.Cu) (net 16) (status 10))
 (segment (start 52.65 37.900001) (end 52.800001 37.75) (width 0.55) (layer F.Cu) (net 16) (status 30))
 (segment (start 51.15 46.45) (end 52.65 44.95) (width 0.55) (layer F.Cu) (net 16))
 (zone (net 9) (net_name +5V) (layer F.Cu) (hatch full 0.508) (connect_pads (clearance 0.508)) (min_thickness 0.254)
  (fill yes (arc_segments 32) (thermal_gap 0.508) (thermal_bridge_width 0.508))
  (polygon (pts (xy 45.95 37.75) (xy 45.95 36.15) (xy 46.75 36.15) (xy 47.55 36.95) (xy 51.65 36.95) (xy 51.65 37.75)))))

